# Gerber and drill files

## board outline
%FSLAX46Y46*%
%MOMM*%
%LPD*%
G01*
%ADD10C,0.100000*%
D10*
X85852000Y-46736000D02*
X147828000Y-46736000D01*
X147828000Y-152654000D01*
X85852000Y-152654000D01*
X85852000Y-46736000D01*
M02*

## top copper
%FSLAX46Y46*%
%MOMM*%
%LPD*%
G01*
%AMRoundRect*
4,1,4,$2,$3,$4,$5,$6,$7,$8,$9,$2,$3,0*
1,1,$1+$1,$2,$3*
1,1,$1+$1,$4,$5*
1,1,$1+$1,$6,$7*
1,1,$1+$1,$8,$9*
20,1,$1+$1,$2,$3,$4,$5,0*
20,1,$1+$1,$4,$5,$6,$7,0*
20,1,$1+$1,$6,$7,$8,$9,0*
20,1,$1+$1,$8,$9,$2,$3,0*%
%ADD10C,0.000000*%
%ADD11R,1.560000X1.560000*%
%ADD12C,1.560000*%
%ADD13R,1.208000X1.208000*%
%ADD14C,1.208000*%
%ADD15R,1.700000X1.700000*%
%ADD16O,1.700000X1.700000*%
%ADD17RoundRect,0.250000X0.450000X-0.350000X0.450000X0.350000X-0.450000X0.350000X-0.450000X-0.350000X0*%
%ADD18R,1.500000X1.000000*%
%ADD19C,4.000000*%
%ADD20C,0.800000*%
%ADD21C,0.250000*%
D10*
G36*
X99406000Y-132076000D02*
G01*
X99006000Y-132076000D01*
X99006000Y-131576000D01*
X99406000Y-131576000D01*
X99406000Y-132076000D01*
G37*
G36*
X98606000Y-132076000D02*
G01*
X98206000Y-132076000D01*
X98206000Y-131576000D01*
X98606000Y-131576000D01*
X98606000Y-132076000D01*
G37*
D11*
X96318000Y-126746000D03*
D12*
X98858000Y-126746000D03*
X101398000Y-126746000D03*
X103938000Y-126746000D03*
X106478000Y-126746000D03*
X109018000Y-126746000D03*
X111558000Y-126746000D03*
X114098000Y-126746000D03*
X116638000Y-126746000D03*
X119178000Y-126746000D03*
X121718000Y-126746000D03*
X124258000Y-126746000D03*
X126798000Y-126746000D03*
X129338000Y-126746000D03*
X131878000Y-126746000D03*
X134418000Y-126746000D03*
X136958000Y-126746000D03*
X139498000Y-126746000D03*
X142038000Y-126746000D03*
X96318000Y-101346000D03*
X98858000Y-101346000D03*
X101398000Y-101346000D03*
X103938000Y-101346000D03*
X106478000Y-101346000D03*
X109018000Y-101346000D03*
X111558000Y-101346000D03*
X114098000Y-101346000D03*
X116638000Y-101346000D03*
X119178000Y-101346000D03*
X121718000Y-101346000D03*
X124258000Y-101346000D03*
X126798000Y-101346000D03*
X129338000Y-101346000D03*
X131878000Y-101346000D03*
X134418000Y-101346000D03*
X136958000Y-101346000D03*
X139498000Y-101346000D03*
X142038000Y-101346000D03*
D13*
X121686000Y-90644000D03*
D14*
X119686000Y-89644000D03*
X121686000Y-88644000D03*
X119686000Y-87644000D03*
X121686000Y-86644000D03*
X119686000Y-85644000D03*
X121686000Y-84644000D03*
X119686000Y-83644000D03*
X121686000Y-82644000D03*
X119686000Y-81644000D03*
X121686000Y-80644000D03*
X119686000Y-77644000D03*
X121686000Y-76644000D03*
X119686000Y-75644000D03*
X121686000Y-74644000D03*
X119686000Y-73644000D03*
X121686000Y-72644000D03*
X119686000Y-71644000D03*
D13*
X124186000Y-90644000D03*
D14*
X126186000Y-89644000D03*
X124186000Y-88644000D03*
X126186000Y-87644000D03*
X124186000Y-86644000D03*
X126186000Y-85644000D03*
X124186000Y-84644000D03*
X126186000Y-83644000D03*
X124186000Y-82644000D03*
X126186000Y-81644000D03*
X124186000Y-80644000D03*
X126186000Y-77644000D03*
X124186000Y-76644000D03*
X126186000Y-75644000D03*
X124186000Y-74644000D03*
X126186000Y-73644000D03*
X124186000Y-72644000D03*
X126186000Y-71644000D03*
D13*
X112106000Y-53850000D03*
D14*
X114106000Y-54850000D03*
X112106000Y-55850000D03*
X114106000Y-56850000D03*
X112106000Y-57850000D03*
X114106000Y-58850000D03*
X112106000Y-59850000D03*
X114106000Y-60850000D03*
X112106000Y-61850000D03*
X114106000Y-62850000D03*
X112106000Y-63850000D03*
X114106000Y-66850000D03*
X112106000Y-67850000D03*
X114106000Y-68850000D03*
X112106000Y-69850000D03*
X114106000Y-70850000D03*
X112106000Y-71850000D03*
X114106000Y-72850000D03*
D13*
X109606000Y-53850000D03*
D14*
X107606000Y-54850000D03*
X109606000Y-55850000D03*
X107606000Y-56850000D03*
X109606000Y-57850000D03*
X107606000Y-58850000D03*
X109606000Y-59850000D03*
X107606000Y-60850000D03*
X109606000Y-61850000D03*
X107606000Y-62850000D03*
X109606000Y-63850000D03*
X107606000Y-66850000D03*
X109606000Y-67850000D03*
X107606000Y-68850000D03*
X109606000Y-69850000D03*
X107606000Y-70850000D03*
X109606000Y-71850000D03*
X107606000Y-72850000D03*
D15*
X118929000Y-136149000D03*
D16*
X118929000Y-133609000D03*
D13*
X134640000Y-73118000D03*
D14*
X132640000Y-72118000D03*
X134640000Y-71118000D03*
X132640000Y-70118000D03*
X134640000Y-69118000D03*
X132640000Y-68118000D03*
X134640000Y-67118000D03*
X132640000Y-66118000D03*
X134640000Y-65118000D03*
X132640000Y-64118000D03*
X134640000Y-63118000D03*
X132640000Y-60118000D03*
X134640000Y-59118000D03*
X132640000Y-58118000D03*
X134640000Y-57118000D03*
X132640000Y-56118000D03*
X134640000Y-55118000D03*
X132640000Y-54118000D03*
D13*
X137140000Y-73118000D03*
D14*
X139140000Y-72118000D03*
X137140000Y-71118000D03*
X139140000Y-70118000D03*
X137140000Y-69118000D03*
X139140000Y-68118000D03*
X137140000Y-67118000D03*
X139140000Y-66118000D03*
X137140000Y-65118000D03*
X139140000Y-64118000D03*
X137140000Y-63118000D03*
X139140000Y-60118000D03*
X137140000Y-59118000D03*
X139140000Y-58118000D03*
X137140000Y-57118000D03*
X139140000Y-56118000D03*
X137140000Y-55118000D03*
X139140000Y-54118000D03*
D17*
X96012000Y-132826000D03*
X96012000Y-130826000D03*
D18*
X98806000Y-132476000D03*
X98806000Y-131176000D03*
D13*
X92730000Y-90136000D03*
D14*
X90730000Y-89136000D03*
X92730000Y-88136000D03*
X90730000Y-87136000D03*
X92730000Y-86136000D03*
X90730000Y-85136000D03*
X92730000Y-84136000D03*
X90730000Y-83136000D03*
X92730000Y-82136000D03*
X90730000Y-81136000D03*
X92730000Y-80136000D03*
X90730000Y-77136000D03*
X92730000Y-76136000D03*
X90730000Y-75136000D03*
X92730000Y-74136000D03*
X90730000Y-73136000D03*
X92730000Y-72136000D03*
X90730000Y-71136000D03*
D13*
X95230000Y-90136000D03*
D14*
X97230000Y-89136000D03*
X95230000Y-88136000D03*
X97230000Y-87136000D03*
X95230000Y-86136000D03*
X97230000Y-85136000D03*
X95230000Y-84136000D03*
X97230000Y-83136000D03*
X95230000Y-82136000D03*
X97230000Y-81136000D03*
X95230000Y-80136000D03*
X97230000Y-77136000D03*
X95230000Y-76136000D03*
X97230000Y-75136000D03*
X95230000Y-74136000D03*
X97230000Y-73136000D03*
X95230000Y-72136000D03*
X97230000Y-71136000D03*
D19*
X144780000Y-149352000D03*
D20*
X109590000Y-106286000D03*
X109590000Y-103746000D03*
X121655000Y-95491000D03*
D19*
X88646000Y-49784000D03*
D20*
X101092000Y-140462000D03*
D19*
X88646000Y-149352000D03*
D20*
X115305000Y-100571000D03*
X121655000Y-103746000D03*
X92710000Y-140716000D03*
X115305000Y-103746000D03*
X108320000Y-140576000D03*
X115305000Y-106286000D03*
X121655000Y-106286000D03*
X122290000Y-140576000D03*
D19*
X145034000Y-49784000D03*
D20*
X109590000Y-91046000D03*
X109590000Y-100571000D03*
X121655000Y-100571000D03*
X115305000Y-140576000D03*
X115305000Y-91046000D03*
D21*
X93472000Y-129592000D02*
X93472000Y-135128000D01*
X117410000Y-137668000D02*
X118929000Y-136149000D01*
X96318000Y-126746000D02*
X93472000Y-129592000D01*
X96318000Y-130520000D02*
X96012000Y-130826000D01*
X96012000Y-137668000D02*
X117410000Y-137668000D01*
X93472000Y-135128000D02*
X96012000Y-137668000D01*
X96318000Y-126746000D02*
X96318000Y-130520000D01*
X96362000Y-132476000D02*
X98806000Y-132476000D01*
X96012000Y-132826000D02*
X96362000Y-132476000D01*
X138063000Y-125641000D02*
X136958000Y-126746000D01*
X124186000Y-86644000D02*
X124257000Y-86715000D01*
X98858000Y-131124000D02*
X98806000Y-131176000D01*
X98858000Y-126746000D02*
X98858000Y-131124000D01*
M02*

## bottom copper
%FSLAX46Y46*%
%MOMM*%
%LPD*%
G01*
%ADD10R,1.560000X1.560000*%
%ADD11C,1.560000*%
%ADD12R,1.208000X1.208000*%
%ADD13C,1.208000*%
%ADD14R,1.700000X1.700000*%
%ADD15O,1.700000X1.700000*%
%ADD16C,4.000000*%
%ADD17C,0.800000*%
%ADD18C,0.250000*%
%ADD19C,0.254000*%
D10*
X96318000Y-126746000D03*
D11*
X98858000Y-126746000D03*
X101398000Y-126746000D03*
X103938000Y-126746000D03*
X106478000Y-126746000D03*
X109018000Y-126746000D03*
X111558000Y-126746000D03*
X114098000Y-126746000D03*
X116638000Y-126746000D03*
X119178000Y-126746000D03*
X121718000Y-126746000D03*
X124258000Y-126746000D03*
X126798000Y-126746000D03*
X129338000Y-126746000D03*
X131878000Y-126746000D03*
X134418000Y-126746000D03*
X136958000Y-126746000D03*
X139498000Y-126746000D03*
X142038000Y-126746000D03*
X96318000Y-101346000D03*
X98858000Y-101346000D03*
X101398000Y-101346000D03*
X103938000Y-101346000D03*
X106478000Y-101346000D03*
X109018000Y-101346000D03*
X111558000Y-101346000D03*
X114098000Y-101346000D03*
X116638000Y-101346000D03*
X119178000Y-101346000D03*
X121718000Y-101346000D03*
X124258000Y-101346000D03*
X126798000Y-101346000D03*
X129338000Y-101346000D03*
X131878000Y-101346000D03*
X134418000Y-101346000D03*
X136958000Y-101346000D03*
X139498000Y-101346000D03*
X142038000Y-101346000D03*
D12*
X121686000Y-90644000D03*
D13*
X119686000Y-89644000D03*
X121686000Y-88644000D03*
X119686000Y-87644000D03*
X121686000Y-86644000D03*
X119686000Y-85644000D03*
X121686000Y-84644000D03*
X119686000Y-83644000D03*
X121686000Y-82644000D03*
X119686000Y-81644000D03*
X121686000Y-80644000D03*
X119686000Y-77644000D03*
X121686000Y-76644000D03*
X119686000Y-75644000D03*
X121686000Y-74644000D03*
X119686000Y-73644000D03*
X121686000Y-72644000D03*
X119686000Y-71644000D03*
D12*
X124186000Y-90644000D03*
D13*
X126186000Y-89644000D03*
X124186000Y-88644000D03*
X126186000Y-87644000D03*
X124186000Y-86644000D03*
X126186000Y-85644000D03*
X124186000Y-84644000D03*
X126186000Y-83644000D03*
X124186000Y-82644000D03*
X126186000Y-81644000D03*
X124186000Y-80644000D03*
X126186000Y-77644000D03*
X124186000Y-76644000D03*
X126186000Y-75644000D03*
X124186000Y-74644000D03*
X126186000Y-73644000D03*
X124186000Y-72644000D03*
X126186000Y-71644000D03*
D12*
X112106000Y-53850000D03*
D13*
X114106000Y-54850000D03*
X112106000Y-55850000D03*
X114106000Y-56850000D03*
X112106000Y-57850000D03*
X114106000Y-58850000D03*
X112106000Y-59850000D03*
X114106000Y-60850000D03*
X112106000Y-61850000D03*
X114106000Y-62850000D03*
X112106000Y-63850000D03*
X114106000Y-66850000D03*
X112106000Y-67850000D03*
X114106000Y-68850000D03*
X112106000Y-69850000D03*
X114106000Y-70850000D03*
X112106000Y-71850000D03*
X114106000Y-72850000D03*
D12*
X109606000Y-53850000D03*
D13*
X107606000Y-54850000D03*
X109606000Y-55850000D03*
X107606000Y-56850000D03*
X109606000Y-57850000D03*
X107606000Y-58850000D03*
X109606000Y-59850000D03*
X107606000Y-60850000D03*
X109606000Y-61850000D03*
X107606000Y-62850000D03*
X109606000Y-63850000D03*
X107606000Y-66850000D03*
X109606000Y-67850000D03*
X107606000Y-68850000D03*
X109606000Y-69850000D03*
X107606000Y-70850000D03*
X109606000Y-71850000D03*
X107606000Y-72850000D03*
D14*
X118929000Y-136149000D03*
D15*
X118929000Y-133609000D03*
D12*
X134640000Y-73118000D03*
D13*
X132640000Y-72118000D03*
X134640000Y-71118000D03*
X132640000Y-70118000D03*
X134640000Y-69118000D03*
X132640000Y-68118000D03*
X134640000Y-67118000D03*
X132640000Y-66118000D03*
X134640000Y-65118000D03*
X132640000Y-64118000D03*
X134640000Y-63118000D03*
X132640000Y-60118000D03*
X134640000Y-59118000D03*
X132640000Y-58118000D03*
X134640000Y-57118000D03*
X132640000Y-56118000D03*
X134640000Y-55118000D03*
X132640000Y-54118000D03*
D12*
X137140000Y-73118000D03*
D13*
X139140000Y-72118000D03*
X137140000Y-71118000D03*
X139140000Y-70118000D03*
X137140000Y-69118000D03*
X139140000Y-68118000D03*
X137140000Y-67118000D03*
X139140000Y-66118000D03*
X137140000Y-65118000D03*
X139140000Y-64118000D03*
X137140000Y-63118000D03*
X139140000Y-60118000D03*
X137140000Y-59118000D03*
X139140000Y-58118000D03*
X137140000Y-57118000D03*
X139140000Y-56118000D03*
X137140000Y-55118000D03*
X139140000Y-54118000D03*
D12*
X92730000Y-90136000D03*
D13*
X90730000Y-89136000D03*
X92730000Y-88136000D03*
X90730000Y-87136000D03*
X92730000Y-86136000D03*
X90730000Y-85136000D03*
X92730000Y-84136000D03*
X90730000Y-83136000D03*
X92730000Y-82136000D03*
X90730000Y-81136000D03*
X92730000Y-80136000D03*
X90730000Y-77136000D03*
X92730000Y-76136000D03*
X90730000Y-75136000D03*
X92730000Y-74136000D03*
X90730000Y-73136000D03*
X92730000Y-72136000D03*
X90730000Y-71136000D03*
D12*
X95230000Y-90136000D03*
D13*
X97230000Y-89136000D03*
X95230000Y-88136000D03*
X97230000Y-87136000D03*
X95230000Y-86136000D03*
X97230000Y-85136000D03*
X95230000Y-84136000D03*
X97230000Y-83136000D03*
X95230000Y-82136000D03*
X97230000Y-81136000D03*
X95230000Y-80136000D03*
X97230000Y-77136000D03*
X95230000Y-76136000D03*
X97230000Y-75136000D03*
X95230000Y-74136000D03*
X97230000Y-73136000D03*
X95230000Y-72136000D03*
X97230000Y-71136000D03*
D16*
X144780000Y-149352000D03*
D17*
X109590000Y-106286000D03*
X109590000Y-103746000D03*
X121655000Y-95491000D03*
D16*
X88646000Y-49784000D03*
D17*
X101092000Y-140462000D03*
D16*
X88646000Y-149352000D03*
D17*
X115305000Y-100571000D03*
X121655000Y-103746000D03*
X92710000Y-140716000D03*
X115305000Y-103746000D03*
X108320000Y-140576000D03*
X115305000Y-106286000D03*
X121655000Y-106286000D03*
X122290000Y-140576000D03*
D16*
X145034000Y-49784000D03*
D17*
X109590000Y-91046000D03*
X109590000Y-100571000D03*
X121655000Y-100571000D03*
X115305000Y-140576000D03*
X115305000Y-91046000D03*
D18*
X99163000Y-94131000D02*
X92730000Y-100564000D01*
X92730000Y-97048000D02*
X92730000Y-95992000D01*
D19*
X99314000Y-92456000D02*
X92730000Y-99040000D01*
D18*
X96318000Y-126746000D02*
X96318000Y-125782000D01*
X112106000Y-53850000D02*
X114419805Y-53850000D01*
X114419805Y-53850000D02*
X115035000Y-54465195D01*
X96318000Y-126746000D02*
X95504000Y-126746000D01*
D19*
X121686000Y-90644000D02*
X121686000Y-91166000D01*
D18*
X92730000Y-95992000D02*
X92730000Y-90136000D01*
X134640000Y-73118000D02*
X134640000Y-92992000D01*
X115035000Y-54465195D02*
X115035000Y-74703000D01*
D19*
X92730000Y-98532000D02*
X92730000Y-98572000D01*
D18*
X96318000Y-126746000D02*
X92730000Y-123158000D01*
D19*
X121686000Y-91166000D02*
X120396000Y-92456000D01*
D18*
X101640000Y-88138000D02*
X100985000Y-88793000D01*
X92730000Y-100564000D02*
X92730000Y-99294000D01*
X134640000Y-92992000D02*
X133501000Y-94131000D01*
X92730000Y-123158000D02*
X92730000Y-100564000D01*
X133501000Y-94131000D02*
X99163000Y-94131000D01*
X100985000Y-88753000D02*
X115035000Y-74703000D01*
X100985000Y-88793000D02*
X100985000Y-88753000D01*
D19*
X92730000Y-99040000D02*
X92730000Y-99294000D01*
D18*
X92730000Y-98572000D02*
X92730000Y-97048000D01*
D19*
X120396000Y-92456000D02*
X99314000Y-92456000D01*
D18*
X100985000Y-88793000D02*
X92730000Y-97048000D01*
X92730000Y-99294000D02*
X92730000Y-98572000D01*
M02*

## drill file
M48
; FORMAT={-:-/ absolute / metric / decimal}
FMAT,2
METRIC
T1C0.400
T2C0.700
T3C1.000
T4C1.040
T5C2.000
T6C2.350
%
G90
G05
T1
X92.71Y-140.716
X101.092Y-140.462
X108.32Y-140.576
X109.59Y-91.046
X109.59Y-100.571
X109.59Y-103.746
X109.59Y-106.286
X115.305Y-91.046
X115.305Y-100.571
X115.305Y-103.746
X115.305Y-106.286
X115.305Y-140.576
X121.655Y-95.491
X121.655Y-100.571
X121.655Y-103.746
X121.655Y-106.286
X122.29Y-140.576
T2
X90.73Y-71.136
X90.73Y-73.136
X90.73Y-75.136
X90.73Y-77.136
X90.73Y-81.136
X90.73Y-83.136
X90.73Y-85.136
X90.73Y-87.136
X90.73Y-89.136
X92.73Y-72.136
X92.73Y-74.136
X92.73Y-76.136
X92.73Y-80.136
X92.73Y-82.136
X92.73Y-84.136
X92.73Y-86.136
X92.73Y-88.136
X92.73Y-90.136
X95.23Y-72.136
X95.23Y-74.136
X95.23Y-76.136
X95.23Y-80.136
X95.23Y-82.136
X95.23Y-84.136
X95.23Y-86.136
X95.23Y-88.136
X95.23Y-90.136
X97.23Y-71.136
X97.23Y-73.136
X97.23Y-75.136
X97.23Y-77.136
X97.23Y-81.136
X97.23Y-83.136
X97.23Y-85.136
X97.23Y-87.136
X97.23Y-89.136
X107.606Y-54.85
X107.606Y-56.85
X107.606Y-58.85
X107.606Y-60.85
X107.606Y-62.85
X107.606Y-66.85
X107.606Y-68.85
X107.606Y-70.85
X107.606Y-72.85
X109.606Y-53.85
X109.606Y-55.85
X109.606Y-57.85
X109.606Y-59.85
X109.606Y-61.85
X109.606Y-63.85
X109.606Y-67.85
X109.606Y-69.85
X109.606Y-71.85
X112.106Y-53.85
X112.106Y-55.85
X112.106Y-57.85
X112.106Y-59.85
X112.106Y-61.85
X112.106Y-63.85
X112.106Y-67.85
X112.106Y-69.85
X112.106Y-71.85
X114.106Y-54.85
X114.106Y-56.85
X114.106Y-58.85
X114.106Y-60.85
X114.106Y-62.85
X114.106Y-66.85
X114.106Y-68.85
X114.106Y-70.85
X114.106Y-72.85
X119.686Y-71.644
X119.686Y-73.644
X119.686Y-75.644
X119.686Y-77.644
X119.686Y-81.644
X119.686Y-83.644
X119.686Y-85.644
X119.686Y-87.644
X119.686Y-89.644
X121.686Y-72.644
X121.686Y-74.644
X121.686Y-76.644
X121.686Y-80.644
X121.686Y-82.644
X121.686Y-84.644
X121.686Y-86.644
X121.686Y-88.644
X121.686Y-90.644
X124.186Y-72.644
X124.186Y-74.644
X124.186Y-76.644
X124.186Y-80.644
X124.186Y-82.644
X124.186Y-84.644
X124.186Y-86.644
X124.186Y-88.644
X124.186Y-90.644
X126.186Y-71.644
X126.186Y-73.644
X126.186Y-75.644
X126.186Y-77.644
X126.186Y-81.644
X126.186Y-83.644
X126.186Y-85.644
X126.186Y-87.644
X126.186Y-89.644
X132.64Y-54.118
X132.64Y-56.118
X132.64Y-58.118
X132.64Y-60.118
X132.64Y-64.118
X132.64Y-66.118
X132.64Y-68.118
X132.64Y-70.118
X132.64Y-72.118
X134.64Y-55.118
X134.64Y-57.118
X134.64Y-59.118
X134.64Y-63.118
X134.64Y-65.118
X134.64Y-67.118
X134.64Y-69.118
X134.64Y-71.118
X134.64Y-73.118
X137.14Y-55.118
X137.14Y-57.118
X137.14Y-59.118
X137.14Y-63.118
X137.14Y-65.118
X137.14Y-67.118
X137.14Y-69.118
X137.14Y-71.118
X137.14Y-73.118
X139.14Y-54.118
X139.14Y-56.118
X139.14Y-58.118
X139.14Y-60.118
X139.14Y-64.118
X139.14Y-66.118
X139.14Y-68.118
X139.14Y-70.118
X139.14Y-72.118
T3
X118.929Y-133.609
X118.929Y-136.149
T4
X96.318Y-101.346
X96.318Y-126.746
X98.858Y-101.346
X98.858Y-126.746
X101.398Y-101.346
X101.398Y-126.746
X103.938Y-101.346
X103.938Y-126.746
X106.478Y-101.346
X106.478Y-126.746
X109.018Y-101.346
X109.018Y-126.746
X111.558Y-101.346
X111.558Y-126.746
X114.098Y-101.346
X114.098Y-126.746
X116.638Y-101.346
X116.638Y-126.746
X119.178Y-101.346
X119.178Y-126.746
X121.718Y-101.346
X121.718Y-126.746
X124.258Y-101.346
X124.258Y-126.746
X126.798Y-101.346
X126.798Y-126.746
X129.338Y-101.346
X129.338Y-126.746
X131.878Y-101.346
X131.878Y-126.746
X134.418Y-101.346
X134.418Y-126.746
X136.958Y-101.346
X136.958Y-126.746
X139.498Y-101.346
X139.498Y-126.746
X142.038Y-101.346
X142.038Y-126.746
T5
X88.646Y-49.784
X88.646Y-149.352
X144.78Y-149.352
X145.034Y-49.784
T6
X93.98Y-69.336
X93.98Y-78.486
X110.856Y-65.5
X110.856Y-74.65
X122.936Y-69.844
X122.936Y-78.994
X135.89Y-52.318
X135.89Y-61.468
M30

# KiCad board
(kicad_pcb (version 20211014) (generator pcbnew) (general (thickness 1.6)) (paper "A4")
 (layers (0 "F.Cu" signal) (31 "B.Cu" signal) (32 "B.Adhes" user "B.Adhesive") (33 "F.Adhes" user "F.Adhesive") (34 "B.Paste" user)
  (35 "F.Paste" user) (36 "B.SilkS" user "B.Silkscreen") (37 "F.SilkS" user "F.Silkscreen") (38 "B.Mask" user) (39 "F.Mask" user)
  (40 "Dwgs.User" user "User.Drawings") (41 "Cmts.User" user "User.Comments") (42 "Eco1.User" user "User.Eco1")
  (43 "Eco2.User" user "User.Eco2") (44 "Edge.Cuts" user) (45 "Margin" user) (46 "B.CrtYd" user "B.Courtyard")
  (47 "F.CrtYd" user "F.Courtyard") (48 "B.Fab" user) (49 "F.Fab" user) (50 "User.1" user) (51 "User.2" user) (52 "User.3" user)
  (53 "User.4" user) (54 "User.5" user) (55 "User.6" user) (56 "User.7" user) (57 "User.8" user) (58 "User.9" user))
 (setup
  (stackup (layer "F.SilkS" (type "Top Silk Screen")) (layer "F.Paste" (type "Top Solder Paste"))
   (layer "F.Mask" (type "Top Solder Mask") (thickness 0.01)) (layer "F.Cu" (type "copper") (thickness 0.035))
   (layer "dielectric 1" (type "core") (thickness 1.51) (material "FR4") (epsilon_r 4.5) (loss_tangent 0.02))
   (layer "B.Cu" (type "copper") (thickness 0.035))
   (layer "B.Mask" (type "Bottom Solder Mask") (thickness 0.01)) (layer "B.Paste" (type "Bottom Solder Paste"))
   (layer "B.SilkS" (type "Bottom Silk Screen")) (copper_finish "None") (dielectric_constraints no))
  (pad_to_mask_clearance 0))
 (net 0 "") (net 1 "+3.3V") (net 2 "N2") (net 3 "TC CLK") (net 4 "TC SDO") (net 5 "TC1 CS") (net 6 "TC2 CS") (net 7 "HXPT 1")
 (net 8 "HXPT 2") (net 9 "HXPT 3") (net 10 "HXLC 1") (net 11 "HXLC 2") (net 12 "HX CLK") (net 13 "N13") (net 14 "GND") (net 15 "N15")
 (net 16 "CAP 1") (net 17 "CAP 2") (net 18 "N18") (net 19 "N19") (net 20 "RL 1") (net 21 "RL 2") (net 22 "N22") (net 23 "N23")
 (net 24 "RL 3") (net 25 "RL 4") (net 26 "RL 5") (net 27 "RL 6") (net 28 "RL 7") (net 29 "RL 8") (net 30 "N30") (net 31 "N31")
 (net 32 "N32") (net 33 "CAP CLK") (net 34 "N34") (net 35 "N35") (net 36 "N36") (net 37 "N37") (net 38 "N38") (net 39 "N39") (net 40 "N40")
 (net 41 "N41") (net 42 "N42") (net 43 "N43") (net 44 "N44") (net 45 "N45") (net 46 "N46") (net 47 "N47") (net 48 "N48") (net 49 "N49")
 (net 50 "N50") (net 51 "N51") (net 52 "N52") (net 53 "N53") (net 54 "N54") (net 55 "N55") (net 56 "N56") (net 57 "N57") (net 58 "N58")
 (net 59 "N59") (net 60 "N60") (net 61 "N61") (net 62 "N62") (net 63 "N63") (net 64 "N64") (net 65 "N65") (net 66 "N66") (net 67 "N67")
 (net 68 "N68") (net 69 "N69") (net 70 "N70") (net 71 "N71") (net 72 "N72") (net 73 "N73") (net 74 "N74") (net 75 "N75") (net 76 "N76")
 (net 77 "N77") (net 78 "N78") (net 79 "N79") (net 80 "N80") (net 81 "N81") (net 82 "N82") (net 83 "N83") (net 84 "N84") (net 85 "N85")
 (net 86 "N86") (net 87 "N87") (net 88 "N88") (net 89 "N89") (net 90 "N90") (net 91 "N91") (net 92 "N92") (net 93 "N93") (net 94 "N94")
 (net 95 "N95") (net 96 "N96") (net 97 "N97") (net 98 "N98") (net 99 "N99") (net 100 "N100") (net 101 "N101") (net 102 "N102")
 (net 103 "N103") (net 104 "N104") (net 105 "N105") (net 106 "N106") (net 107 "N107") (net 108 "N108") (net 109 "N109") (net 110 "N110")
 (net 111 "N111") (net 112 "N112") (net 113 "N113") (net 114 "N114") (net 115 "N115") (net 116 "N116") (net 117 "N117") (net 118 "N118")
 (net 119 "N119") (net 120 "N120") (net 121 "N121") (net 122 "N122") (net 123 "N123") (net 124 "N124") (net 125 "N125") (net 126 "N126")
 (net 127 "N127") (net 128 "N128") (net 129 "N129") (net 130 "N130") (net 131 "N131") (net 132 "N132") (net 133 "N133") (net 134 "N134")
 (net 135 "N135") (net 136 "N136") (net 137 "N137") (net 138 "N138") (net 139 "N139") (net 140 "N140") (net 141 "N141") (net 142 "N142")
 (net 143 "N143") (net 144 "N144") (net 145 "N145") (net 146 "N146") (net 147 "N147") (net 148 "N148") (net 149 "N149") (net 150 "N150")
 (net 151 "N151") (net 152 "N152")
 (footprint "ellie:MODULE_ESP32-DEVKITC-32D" (layer "F.Cu") (at 116.078 114.046 90)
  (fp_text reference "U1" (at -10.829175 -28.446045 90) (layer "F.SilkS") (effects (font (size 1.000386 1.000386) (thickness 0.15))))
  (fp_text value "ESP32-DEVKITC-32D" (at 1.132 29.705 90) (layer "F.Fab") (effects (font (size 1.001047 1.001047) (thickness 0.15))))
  (pad "1" thru_hole rect locked (at -12.7 -19.76 90) (size 1.56 1.56) (drill 1.04) (layers *.Cu *.Mask) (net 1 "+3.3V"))
  (pad "2" thru_hole circle locked (at -12.7 -17.22 90) (size 1.56 1.56) (drill 1.04) (layers *.Cu *.Mask) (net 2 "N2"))
  (pad "3" thru_hole circle locked (at -12.7 -14.68 90) (size 1.56 1.56) (drill 1.04) (layers *.Cu *.Mask) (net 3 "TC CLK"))
  (pad "4" thru_hole circle locked (at -12.7 -12.14 90) (size 1.56 1.56) (drill 1.04) (layers *.Cu *.Mask) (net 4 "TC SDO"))
  (pad "5" thru_hole circle locked (at -12.7 -9.6 90) (size 1.56 1.56) (drill 1.04) (layers *.Cu *.Mask) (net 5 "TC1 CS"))
  (pad "6" thru_hole circle locked (at -12.7 -7.06 90) (size 1.56 1.56) (drill 1.04) (layers *.Cu *.Mask) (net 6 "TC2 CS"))
  (pad "7" thru_hole circle locked (at -12.7 -4.52 90) (size 1.56 1.56) (drill 1.04) (layers *.Cu *.Mask) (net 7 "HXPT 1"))
  (pad "8" thru_hole circle locked (at -12.7 -1.98 90) (size 1.56 1.56) (drill 1.04) (layers *.Cu *.Mask) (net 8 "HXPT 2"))
  (pad "9" thru_hole circle locked (at -12.7 0.56 90) (size 1.56 1.56) (drill 1.04) (layers *.Cu *.Mask) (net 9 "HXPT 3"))
  (pad "10" thru_hole circle locked (at -12.7 3.1 90) (size 1.56 1.56) (drill 1.04) (layers *.Cu *.Mask) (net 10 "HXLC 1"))
  (pad "11" thru_hole circle locked (at -12.7 5.64 90) (size 1.56 1.56) (drill 1.04) (layers *.Cu *.Mask) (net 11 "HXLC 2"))
  (pad "12" thru_hole circle locked (at -12.7 8.18 90) (size 1.56 1.56) (drill 1.04) (layers *.Cu *.Mask) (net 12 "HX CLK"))
  (pad "13" thru_hole circle locked (at -12.7 10.72 90) (size 1.56 1.56) (drill 1.04) (layers *.Cu *.Mask) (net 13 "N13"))
  (pad "14" thru_hole circle locked (at -12.7 13.26 90) (size 1.56 1.56) (drill 1.04) (layers *.Cu *.Mask) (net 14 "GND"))
  (pad "15" thru_hole circle locked (at -12.7 15.8 90) (size 1.56 1.56) (drill 1.04) (layers *.Cu *.Mask) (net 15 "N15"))
  (pad "16" thru_hole circle locked (at -12.7 18.34 90) (size 1.56 1.56) (drill 1.04) (layers *.Cu *.Mask) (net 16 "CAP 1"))
  (pad "17" thru_hole circle locked (at -12.7 20.88 90) (size 1.56 1.56) (drill 1.04) (layers *.Cu *.Mask) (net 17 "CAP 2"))
  (pad "18" thru_hole circle locked (at -12.7 23.42 90) (size 1.56 1.56) (drill 1.04) (layers *.Cu *.Mask) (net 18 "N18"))
  (pad "19" thru_hole circle locked (at -12.7 25.96 90) (size 1.56 1.56) (drill 1.04) (layers *.Cu *.Mask) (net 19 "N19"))
  (pad "20" thru_hole circle locked (at 12.7 -19.76 90) (size 1.56 1.56) (drill 1.04) (layers *.Cu *.Mask) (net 14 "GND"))
  (pad "21" thru_hole circle locked (at 12.7 -17.22 90) (size 1.56 1.56) (drill 1.04) (layers *.Cu *.Mask) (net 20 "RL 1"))
  (pad "22" thru_hole circle locked (at 12.7 -14.68 90) (size 1.56 1.56) (drill 1.04) (layers *.Cu *.Mask) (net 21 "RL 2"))
  (pad "23" thru_hole circle locked (at 12.7 -12.14 90) (size 1.56 1.56) (drill 1.04) (layers *.Cu *.Mask) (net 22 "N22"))
  (pad "24" thru_hole circle locked (at 12.7 -9.6 90) (size 1.56 1.56) (drill 1.04) (layers *.Cu *.Mask) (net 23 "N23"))
  (pad "25" thru_hole circle locked (at 12.7 -7.06 90) (size 1.56 1.56) (drill 1.04) (layers *.Cu *.Mask) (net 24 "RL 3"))
  (pad "26" thru_hole circle locked (at 12.7 -4.52 90) (size 1.56 1.56) (drill 1.04) (layers *.Cu *.Mask) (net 14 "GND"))
  (pad "27" thru_hole circle locked (at 12.7 -1.98 90) (size 1.56 1.56) (drill 1.04) (layers *.Cu *.Mask) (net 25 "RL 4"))
  (pad "28" thru_hole circle locked (at 12.7 0.56 90) (size 1.56 1.56) (drill 1.04) (layers *.Cu *.Mask) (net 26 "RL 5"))
  (pad "29" thru_hole circle locked (at 12.7 3.1 90) (size 1.56 1.56) (drill 1.04) (layers *.Cu *.Mask) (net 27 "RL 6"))
  (pad "30" thru_hole circle locked (at 12.7 5.64 90) (size 1.56 1.56) (drill 1.04) (layers *.Cu *.Mask) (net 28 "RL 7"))
  (pad "31" thru_hole circle locked (at 12.7 8.18 90) (size 1.56 1.56) (drill 1.04) (layers *.Cu *.Mask) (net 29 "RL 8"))
  (pad "32" thru_hole circle locked (at 12.7 10.72 90) (size 1.56 1.56) (drill 1.04) (layers *.Cu *.Mask) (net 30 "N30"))
  (pad "33" thru_hole circle locked (at 12.7 13.26 90) (size 1.56 1.56) (drill 1.04) (layers *.Cu *.Mask) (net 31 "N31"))
  (pad "34" thru_hole circle locked (at 12.7 15.8 90) (size 1.56 1.56) (drill 1.04) (layers *.Cu *.Mask) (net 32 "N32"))
  (pad "35" thru_hole circle locked (at 12.7 18.34 90) (size 1.56 1.56) (drill 1.04) (layers *.Cu *.Mask) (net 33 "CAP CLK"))
  (pad "36" thru_hole circle locked (at 12.7 20.88 90) (size 1.56 1.56) (drill 1.04) (layers *.Cu *.Mask) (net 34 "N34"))
  (pad "37" thru_hole circle locked (at 12.7 23.42 90) (size 1.56 1.56) (drill 1.04) (layers *.Cu *.Mask) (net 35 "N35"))
  (pad "38" thru_hole circle locked (at 12.7 25.96 90) (size 1.56 1.56) (drill 1.04) (layers *.Cu *.Mask) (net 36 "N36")))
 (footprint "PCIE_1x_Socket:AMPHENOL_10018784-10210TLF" (layer "F.Cu") (at 122.936 78.994 90)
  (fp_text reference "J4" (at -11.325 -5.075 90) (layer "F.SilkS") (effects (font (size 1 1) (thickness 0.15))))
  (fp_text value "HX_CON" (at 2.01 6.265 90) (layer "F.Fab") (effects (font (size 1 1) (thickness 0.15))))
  (pad "" np_thru_hole circle locked (at 9.15 0 90) (size 2.35 2.35) (drill 2.35) (layers *.Cu *.Mask))
  (pad "" np_thru_hole circle locked (at 0 0 90) (size 2.35 2.35) (drill 2.35) (layers *.Cu *.Mask))
  (pad "A1" thru_hole rect locked (at -11.65 -1.25 90) (size 1.208 1.208) (drill 0.7) (layers *.Cu *.Mask) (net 1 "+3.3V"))
  (pad "A2" thru_hole circle locked (at -10.65 -3.25 90) (size 1.208 1.208) (drill 0.7) (layers *.Cu *.Mask) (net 14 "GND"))
  (pad "A3" thru_hole circle locked (at -9.65 -1.25 90) (size 1.208 1.208) (drill 0.7) (layers *.Cu *.Mask) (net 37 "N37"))
  (pad "A4" thru_hole circle locked (at -8.65 -3.25 90) (size 1.208 1.208) (drill 0.7) (layers *.Cu *.Mask) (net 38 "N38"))
  (pad "A5" thru_hole circle locked (at -7.65 -1.25 90) (size 1.208 1.208) (drill 0.7) (layers *.Cu *.Mask) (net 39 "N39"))
  (pad "A6" thru_hole circle locked (at -6.65 -3.25 90) (size 1.208 1.208) (drill 0.7) (layers *.Cu *.Mask) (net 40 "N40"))
  (pad "A7" thru_hole circle locked (at -5.65 -1.25 90) (size 1.208 1.208) (drill 0.7) (layers *.Cu *.Mask) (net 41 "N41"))
  (pad "A8" thru_hole circle locked (at -4.65 -3.25 90) (size 1.208 1.208) (drill 0.7) (layers *.Cu *.Mask) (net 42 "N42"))
  (pad "A9" thru_hole circle locked (at -3.65 -1.25 90) (size 1.208 1.208) (drill 0.7) (layers *.Cu *.Mask) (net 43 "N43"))
  (pad "A10" thru_hole circle locked (at -2.65 -3.25 90) (size 1.208 1.208) (drill 0.7) (layers *.Cu *.Mask) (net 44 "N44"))
  (pad "A11" thru_hole circle locked (at -1.65 -1.25 90) (size 1.208 1.208) (drill 0.7) (layers *.Cu *.Mask) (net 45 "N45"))
  (pad "A12" thru_hole circle locked (at 1.35 -3.25 90) (size 1.208 1.208) (drill 0.7) (layers *.Cu *.Mask) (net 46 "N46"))
  (pad "A13" thru_hole circle locked (at 2.35 -1.25 90) (size 1.208 1.208) (drill 0.7) (layers *.Cu *.Mask) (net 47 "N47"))
  (pad "A14" thru_hole circle locked (at 3.35 -3.25 90) (size 1.208 1.208) (drill 0.7) (layers *.Cu *.Mask) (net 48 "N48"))
  (pad "A15" thru_hole circle locked (at 4.35 -1.25 90) (size 1.208 1.208) (drill 0.7) (layers *.Cu *.Mask) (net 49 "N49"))
  (pad "A16" thru_hole circle locked (at 5.35 -3.25 90) (size 1.208 1.208) (drill 0.7) (layers *.Cu *.Mask) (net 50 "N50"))
  (pad "A17" thru_hole circle locked (at 6.35 -1.25 90) (size 1.208 1.208) (drill 0.7) (layers *.Cu *.Mask) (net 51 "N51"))
  (pad "A18" thru_hole circle locked (at 7.35 -3.25 90) (size 1.208 1.208) (drill 0.7) (layers *.Cu *.Mask) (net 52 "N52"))
  (pad "B1" thru_hole rect locked (at -11.65 1.25 90) (size 1.208 1.208) (drill 0.7) (layers *.Cu *.Mask) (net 7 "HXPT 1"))
  (pad "B2" thru_hole circle locked (at -10.65 3.25 90) (size 1.208 1.208) (drill 0.7) (layers *.Cu *.Mask) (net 8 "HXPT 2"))
  (pad "B3" thru_hole circle locked (at -9.65 1.25 90) (size 1.208 1.208) (drill 0.7) (layers *.Cu *.Mask) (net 9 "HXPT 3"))
  (pad "B4" thru_hole circle locked (at -8.65 3.25 90) (size 1.208 1.208) (drill 0.7) (layers *.Cu *.Mask) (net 10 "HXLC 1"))
  (pad "B5" thru_hole circle locked (at -7.65 1.25 90) (size 1.208 1.208) (drill 0.7) (layers *.Cu *.Mask) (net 11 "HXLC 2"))
  (pad "B6" thru_hole circle locked (at -6.65 3.25 90) (size 1.208 1.208) (drill 0.7) (layers *.Cu *.Mask) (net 12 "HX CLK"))
  (pad "B7" thru_hole circle locked (at -5.65 1.25 90) (size 1.208 1.208) (drill 0.7) (layers *.Cu *.Mask) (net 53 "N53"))
  (pad "B8" thru_hole circle locked (at -4.65 3.25 90) (size 1.208 1.208) (drill 0.7) (layers *.Cu *.Mask) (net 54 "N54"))
  (pad "B9" thru_hole circle locked (at -3.65 1.25 90) (size 1.208 1.208) (drill 0.7) (layers *.Cu *.Mask) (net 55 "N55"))
  (pad "B10" thru_hole circle locked (at -2.65 3.25 90) (size 1.208 1.208) (drill 0.7) (layers *.Cu *.Mask) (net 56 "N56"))
  (pad "B11" thru_hole circle locked (at -1.65 1.25 90) (size 1.208 1.208) (drill 0.7) (layers *.Cu *.Mask) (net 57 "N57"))
  (pad "B12" thru_hole circle locked (at 1.35 3.25 90) (size 1.208 1.208) (drill 0.7) (layers *.Cu *.Mask) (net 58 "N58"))
  (pad "B13" thru_hole circle locked (at 2.35 1.25 90) (size 1.208 1.208) (drill 0.7) (layers *.Cu *.Mask) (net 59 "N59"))
  (pad "B14" thru_hole circle locked (at 3.35 3.25 90) (size 1.208 1.208) (drill 0.7) (layers *.Cu *.Mask) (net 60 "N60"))
  (pad "B15" thru_hole circle locked (at 4.35 1.25 90) (size 1.208 1.208) (drill 0.7) (layers *.Cu *.Mask) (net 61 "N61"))
  (pad "B16" thru_hole circle locked (at 5.35 3.25 90) (size 1.208 1.208) (drill 0.7) (layers *.Cu *.Mask) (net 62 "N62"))
  (pad "B17" thru_hole circle locked (at 6.35 1.25 90) (size 1.208 1.208) (drill 0.7) (layers *.Cu *.Mask) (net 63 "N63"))
  (pad "B18" thru_hole circle locked (at 7.35 3.25 90) (size 1.208 1.208) (drill 0.7) (layers *.Cu *.Mask) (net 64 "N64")))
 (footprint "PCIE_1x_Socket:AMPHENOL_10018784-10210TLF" (layer "F.Cu") (at 110.856 65.5 -90)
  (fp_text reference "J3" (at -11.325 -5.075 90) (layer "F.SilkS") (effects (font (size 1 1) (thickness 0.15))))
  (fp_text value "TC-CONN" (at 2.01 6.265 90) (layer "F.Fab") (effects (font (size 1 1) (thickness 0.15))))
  (pad "" np_thru_hole circle locked (at 0 0 270) (size 2.35 2.35) (drill 2.35) (layers *.Cu *.Mask))
  (pad "" np_thru_hole circle locked (at 9.15 0 270) (size 2.35 2.35) (drill 2.35) (layers *.Cu *.Mask))
  (pad "A1" thru_hole rect locked (at -11.65 -1.25 270) (size 1.208 1.208) (drill 0.7) (layers *.Cu *.Mask) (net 1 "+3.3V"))
  (pad "A2" thru_hole circle locked (at -10.65 -3.25 270) (size 1.208 1.208) (drill 0.7) (layers *.Cu *.Mask) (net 14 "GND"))
  (pad "A3" thru_hole circle locked (at -9.65 -1.25 270) (size 1.208 1.208) (drill 0.7) (layers *.Cu *.Mask) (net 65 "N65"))
  (pad "A4" thru_hole circle locked (at -8.65 -3.25 270) (size 1.208 1.208) (drill 0.7) (layers *.Cu *.Mask) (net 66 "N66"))
  (pad "A5" thru_hole circle locked (at -7.65 -1.25 270) (size 1.208 1.208) (drill 0.7) (layers *.Cu *.Mask) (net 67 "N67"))
  (pad "A6" thru_hole circle locked (at -6.65 -3.25 270) (size 1.208 1.208) (drill 0.7) (layers *.Cu *.Mask) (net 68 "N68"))
  (pad "A7" thru_hole circle locked (at -5.65 -1.25 270) (size 1.208 1.208) (drill 0.7) (layers *.Cu *.Mask) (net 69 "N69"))
  (pad "A8" thru_hole circle locked (at -4.65 -3.25 270) (size 1.208 1.208) (drill 0.7) (layers *.Cu *.Mask) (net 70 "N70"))
  (pad "A9" thru_hole circle locked (at -3.65 -1.25 270) (size 1.208 1.208) (drill 0.7) (layers *.Cu *.Mask) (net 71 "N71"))
  (pad "A10" thru_hole circle locked (at -2.65 -3.25 270) (size 1.208 1.208) (drill 0.7) (layers *.Cu *.Mask) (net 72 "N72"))
  (pad "A11" thru_hole circle locked (at -1.65 -1.25 270) (size 1.208 1.208) (drill 0.7) (layers *.Cu *.Mask) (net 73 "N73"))
  (pad "A12" thru_hole circle locked (at 1.35 -3.25 270) (size 1.208 1.208) (drill 0.7) (layers *.Cu *.Mask) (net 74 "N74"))
  (pad "A13" thru_hole circle locked (at 2.35 -1.25 270) (size 1.208 1.208) (drill 0.7) (layers *.Cu *.Mask) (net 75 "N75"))
  (pad "A14" thru_hole circle locked (at 3.35 -3.25 270) (size 1.208 1.208) (drill 0.7) (layers *.Cu *.Mask) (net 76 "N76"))
  (pad "A15" thru_hole circle locked (at 4.35 -1.25 270) (size 1.208 1.208) (drill 0.7) (layers *.Cu *.Mask) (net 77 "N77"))
  (pad "A16" thru_hole circle locked (at 5.35 -3.25 270) (size 1.208 1.208) (drill 0.7) (layers *.Cu *.Mask) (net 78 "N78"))
  (pad "A17" thru_hole circle locked (at 6.35 -1.25 270) (size 1.208 1.208) (drill 0.7) (layers *.Cu *.Mask) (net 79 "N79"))
  (pad "A18" thru_hole circle locked (at 7.35 -3.25 270) (size 1.208 1.208) (drill 0.7) (layers *.Cu *.Mask) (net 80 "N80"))
  (pad "B1" thru_hole rect locked (at -11.65 1.25 270) (size 1.208 1.208) (drill 0.7) (layers *.Cu *.Mask) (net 6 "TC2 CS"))
  (pad "B2" thru_hole circle locked (at -10.65 3.25 270) (size 1.208 1.208) (drill 0.7) (layers *.Cu *.Mask) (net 5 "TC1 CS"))
  (pad "B3" thru_hole circle locked (at -9.65 1.25 270) (size 1.208 1.208) (drill 0.7) (layers *.Cu *.Mask) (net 4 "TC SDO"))
  (pad "B4" thru_hole circle locked (at -8.65 3.25 270) (size 1.208 1.208) (drill 0.7) (layers *.Cu *.Mask) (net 3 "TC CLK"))
  (pad "B5" thru_hole circle locked (at -7.65 1.25 270) (size 1.208 1.208) (drill 0.7) (layers *.Cu *.Mask) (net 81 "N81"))
  (pad "B6" thru_hole circle locked (at -6.65 3.25 270) (size 1.208 1.208) (drill 0.7) (layers *.Cu *.Mask) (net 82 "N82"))
  (pad "B7" thru_hole circle locked (at -5.65 1.25 270) (size 1.208 1.208) (drill 0.7) (layers *.Cu *.Mask) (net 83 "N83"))
  (pad "B8" thru_hole circle locked (at -4.65 3.25 270) (size 1.208 1.208) (drill 0.7) (layers *.Cu *.Mask) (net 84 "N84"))
  (pad "B9" thru_hole circle locked (at -3.65 1.25 270) (size 1.208 1.208) (drill 0.7) (layers *.Cu *.Mask) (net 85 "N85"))
  (pad "B10" thru_hole circle locked (at -2.65 3.25 270) (size 1.208 1.208) (drill 0.7) (layers *.Cu *.Mask) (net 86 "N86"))
  (pad "B11" thru_hole circle locked (at -1.65 1.25 270) (size 1.208 1.208) (drill 0.7) (layers *.Cu *.Mask) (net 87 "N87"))
  (pad "B12" thru_hole circle locked (at 1.35 3.25 270) (size 1.208 1.208) (drill 0.7) (layers *.Cu *.Mask) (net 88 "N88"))
  (pad "B13" thru_hole circle locked (at 2.35 1.25 270) (size 1.208 1.208) (drill 0.7) (layers *.Cu *.Mask) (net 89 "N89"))
  (pad "B14" thru_hole circle locked (at 3.35 3.25 270) (size 1.208 1.208) (drill 0.7) (layers *.Cu *.Mask) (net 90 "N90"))
  (pad "B15" thru_hole circle locked (at 4.35 1.25 270) (size 1.208 1.208) (drill 0.7) (layers *.Cu *.Mask) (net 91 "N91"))
  (pad "B16" thru_hole circle locked (at 5.35 3.25 270) (size 1.208 1.208) (drill 0.7) (layers *.Cu *.Mask) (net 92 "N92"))
  (pad "B17" thru_hole circle locked (at 6.35 1.25 270) (size 1.208 1.208) (drill 0.7) (layers *.Cu *.Mask) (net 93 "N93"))
  (pad "B18" thru_hole circle locked (at 7.35 3.25 270) (size 1.208 1.208) (drill 0.7) (layers *.Cu *.Mask) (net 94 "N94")))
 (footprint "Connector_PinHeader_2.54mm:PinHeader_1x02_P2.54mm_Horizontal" (layer "F.Cu") (at 118.929 136.149 180)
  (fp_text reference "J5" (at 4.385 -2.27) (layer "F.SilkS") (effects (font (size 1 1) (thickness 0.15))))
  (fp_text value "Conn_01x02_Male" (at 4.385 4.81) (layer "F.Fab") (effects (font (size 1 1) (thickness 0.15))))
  (pad "1" thru_hole rect (at 0 0 180) (size 1.7 1.7) (drill 1) (layers *.Cu *.Mask) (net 1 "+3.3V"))
  (pad "2" thru_hole oval (at 0 2.54 180) (size 1.7 1.7) (drill 1) (layers *.Cu *.Mask) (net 14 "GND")))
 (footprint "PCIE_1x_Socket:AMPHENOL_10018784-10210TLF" (layer "F.Cu") (at 135.89 61.468 90)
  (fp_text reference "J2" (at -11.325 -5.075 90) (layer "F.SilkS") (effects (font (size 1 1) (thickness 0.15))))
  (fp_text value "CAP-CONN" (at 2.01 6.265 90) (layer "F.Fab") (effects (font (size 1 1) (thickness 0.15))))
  (pad "" np_thru_hole circle locked (at 9.15 0 90) (size 2.35 2.35) (drill 2.35) (layers *.Cu *.Mask))
  (pad "" np_thru_hole circle locked (at 0 0 90) (size 2.35 2.35) (drill 2.35) (layers *.Cu *.Mask))
  (pad "A1" thru_hole rect locked (at -11.65 -1.25 90) (size 1.208 1.208) (drill 0.7) (layers *.Cu *.Mask) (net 1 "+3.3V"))
  (pad "A2" thru_hole circle locked (at -10.65 -3.25 90) (size 1.208 1.208) (drill 0.7) (layers *.Cu *.Mask) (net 14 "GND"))
  (pad "A3" thru_hole circle locked (at -9.65 -1.25 90) (size 1.208 1.208) (drill 0.7) (layers *.Cu *.Mask) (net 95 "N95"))
  (pad "A4" thru_hole circle locked (at -8.65 -3.25 90) (size 1.208 1.208) (drill 0.7) (layers *.Cu *.Mask) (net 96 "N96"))
  (pad "A5" thru_hole circle locked (at -7.65 -1.25 90) (size 1.208 1.208) (drill 0.7) (layers *.Cu *.Mask) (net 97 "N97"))
  (pad "A6" thru_hole circle locked (at -6.65 -3.25 90) (size 1.208 1.208) (drill 0.7) (layers *.Cu *.Mask) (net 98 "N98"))
  (pad "A7" thru_hole circle locked (at -5.65 -1.25 90) (size 1.208 1.208) (drill 0.7) (layers *.Cu *.Mask) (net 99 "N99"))
  (pad "A8" thru_hole circle locked (at -4.65 -3.25 90) (size 1.208 1.208) (drill 0.7) (layers *.Cu *.Mask) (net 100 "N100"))
  (pad "A9" thru_hole circle locked (at -3.65 -1.25 90) (size 1.208 1.208) (drill 0.7) (layers *.Cu *.Mask) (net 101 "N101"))
  (pad "A10" thru_hole circle locked (at -2.65 -3.25 90) (size 1.208 1.208) (drill 0.7) (layers *.Cu *.Mask) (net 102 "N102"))
  (pad "A11" thru_hole circle locked (at -1.65 -1.25 90) (size 1.208 1.208) (drill 0.7) (layers *.Cu *.Mask) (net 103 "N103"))
  (pad "A12" thru_hole circle locked (at 1.35 -3.25 90) (size 1.208 1.208) (drill 0.7) (layers *.Cu *.Mask) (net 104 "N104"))
  (pad "A13" thru_hole circle locked (at 2.35 -1.25 90) (size 1.208 1.208) (drill 0.7) (layers *.Cu *.Mask) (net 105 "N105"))
  (pad "A14" thru_hole circle locked (at 3.35 -3.25 90) (size 1.208 1.208) (drill 0.7) (layers *.Cu *.Mask) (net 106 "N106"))
  (pad "A15" thru_hole circle locked (at 4.35 -1.25 90) (size 1.208 1.208) (drill 0.7) (layers *.Cu *.Mask) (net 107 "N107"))
  (pad "A16" thru_hole circle locked (at 5.35 -3.25 90) (size 1.208 1.208) (drill 0.7) (layers *.Cu *.Mask) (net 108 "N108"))
  (pad "A17" thru_hole circle locked (at 6.35 -1.25 90) (size 1.208 1.208) (drill 0.7) (layers *.Cu *.Mask) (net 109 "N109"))
  (pad "A18" thru_hole circle locked (at 7.35 -3.25 90) (size 1.208 1.208) (drill 0.7) (layers *.Cu *.Mask) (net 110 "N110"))
  (pad "B1" thru_hole rect locked (at -11.65 1.25 90) (size 1.208 1.208) (drill 0.7) (layers *.Cu *.Mask) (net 16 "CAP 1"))
  (pad "B2" thru_hole circle locked (at -10.65 3.25 90) (size 1.208 1.208) (drill 0.7) (layers *.Cu *.Mask) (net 17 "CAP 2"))
  (pad "B3" thru_hole circle locked (at -9.65 1.25 90) (size 1.208 1.208) (drill 0.7) (layers *.Cu *.Mask) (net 33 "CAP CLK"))
  (pad "B4" thru_hole circle locked (at -8.65 3.25 90) (size 1.208 1.208) (drill 0.7) (layers *.Cu *.Mask) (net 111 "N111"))
  (pad "B5" thru_hole circle locked (at -7.65 1.25 90) (size 1.208 1.208) (drill 0.7) (layers *.Cu *.Mask) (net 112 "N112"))
  (pad "B6" thru_hole circle locked (at -6.65 3.25 90) (size 1.208 1.208) (drill 0.7) (layers *.Cu *.Mask) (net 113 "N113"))
  (pad "B7" thru_hole circle locked (at -5.65 1.25 90) (size 1.208 1.208) (drill 0.7) (layers *.Cu *.Mask) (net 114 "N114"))
  (pad "B8" thru_hole circle locked (at -4.65 3.25 90) (size 1.208 1.208) (drill 0.7) (layers *.Cu *.Mask) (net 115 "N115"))
  (pad "B9" thru_hole circle locked (at -3.65 1.25 90) (size 1.208 1.208) (drill 0.7) (layers *.Cu *.Mask) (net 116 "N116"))
  (pad "B10" thru_hole circle locked (at -2.65 3.25 90) (size 1.208 1.208) (drill 0.7) (layers *.Cu *.Mask) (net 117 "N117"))
  (pad "B11" thru_hole circle locked (at -1.65 1.25 90) (size 1.208 1.208) (drill 0.7) (layers *.Cu *.Mask) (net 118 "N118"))
  (pad "B12" thru_hole circle locked (at 1.35 3.25 90) (size 1.208 1.208) (drill 0.7) (layers *.Cu *.Mask) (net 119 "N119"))
  (pad "B13" thru_hole circle locked (at 2.35 1.25 90) (size 1.208 1.208) (drill 0.7) (layers *.Cu *.Mask) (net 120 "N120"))
  (pad "B14" thru_hole circle locked (at 3.35 3.25 90) (size 1.208 1.208) (drill 0.7) (layers *.Cu *.Mask) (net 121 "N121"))
  (pad "B15" thru_hole circle locked (at 4.35 1.25 90) (size 1.208 1.208) (drill 0.7) (layers *.Cu *.Mask) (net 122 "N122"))
  (pad "B16" thru_hole circle locked (at 5.35 3.25 90) (size 1.208 1.208) (drill 0.7) (layers *.Cu *.Mask) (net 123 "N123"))
  (pad "B17" thru_hole circle locked (at 6.35 1.25 90) (size 1.208 1.208) (drill 0.7) (layers *.Cu *.Mask) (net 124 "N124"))
  (pad "B18" thru_hole circle locked (at 7.35 3.25 90) (size 1.208 1.208) (drill 0.7) (layers *.Cu *.Mask) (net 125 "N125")))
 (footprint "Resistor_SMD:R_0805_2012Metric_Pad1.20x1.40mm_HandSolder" (layer "F.Cu") (at 96.012 131.826 90)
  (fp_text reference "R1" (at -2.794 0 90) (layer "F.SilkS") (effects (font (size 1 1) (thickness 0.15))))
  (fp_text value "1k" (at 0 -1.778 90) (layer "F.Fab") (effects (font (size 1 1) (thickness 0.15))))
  (pad "1" smd roundrect (at -1 0 90) (size 1.2 1.4) (layers "F.Cu" "F.Paste" "F.Mask") (roundrect_rratio 0.208333) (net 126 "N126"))
  (pad "2" smd roundrect (at 1 0 90) (size 1.2 1.4) (layers "F.Cu" "F.Paste" "F.Mask") (roundrect_rratio 0.208333) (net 1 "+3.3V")))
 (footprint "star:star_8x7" (layer "F.Cu") (at 130.302 137.922 90)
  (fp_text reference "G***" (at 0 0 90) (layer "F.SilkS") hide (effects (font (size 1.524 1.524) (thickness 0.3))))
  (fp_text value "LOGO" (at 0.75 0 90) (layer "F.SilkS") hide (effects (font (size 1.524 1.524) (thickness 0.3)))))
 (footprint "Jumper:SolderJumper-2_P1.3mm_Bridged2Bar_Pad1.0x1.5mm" (layer "F.Cu") (at 98.806 131.826 90)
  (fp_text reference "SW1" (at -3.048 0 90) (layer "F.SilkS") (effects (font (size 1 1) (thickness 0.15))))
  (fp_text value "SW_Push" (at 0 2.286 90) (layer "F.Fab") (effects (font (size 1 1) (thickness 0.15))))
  (fp_poly (pts (xy -0.25 0.2) (xy 0.25 0.2) (xy 0.25 0.6) (xy -0.25 0.6)) (layer "F.Cu") (width 0) (fill solid))
  (fp_poly (pts (xy -0.25 -0.6) (xy 0.25 -0.6) (xy 0.25 -0.2) (xy -0.25 -0.2)) (layer "F.Cu") (width 0) (fill solid))
  (pad "1" smd rect (at -0.65 0 90) (size 1 1.5) (layers "F.Cu" "F.Mask") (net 126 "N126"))
  (pad "2" smd rect (at 0.65 0 90) (size 1 1.5) (layers "F.Cu" "F.Mask") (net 2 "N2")))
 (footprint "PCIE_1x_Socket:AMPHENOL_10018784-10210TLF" (layer "F.Cu") (at 93.98 78.486 90)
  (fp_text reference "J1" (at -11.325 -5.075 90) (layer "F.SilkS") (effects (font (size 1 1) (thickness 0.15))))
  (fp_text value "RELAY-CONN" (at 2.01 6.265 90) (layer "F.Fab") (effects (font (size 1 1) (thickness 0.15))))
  (pad "" np_thru_hole circle locked (at 9.15 0 90) (size 2.35 2.35) (drill 2.35) (layers *.Cu *.Mask))
  (pad "" np_thru_hole circle locked (at 0 0 90) (size 2.35 2.35) (drill 2.35) (layers *.Cu *.Mask))
  (pad "A1" thru_hole rect locked (at -11.65 -1.25 90) (size 1.208 1.208) (drill 0.7) (layers *.Cu *.Mask) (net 1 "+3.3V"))
  (pad "A2" thru_hole circle locked (at -10.65 -3.25 90) (size 1.208 1.208) (drill 0.7) (layers *.Cu *.Mask) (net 14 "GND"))
  (pad "A3" thru_hole circle locked (at -9.65 -1.25 90) (size 1.208 1.208) (drill 0.7) (layers *.Cu *.Mask) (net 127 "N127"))
  (pad "A4" thru_hole circle locked (at -8.65 -3.25 90) (size 1.208 1.208) (drill 0.7) (layers *.Cu *.Mask) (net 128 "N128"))
  (pad "A5" thru_hole circle locked (at -7.65 -1.25 90) (size 1.208 1.208) (drill 0.7) (layers *.Cu *.Mask) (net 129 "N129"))
  (pad "A6" thru_hole circle locked (at -6.65 -3.25 90) (size 1.208 1.208) (drill 0.7) (layers *.Cu *.Mask) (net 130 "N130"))
  (pad "A7" thru_hole circle locked (at -5.65 -1.25 90) (size 1.208 1.208) (drill 0.7) (layers *.Cu *.Mask) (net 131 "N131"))
  (pad "A8" thru_hole circle locked (at -4.65 -3.25 90) (size 1.208 1.208) (drill 0.7) (layers *.Cu *.Mask) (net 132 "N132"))
  (pad "A9" thru_hole circle locked (at -3.65 -1.25 90) (size 1.208 1.208) (drill 0.7) (layers *.Cu *.Mask) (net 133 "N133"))
  (pad "A10" thru_hole circle locked (at -2.65 -3.25 90) (size 1.208 1.208) (drill 0.7) (layers *.Cu *.Mask) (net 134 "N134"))
  (pad "A11" thru_hole circle locked (at -1.65 -1.25 90) (size 1.208 1.208) (drill 0.7) (layers *.Cu *.Mask) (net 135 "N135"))
  (pad "A12" thru_hole circle locked (at 1.35 -3.25 90) (size 1.208 1.208) (drill 0.7) (layers *.Cu *.Mask) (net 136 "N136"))
  (pad "A13" thru_hole circle locked (at 2.35 -1.25 90) (size 1.208 1.208) (drill 0.7) (layers *.Cu *.Mask) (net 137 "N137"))
  (pad "A14" thru_hole circle locked (at 3.35 -3.25 90) (size 1.208 1.208) (drill 0.7) (layers *.Cu *.Mask) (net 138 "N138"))
  (pad "A15" thru_hole circle locked (at 4.35 -1.25 90) (size 1.208 1.208) (drill 0.7) (layers *.Cu *.Mask) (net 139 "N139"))
  (pad "A16" thru_hole circle locked (at 5.35 -3.25 90) (size 1.208 1.208) (drill 0.7) (layers *.Cu *.Mask) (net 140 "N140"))
  (pad "A17" thru_hole circle locked (at 6.35 -1.25 90) (size 1.208 1.208) (drill 0.7) (layers *.Cu *.Mask) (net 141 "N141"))
  (pad "A18" thru_hole circle locked (at 7.35 -3.25 90) (size 1.208 1.208) (drill 0.7) (layers *.Cu *.Mask) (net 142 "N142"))
  (pad "B1" thru_hole rect locked (at -11.65 1.25 90) (size 1.208 1.208) (drill 0.7) (layers *.Cu *.Mask) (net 20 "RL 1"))
  (pad "B2" thru_hole circle locked (at -10.65 3.25 90) (size 1.208 1.208) (drill 0.7) (layers *.Cu *.Mask) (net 21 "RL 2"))
  (pad "B3" thru_hole circle locked (at -9.65 1.25 90) (size 1.208 1.208) (drill 0.7) (layers *.Cu *.Mask) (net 24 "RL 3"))
  (pad "B4" thru_hole circle locked (at -8.65 3.25 90) (size 1.208 1.208) (drill 0.7) (layers *.Cu *.Mask) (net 25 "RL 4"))
  (pad "B5" thru_hole circle locked (at -7.65 1.25 90) (size 1.208 1.208) (drill 0.7) (layers *.Cu *.Mask) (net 26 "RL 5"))
  (pad "B6" thru_hole circle locked (at -6.65 3.25 90) (size 1.208 1.208) (drill 0.7) (layers *.Cu *.Mask) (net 27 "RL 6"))
  (pad "B7" thru_hole circle locked (at -5.65 1.25 90) (size 1.208 1.208) (drill 0.7) (layers *.Cu *.Mask) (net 28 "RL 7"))
  (pad "B8" thru_hole circle locked (at -4.65 3.25 90) (size 1.208 1.208) (drill 0.7) (layers *.Cu *.Mask) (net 29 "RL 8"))
  (pad "B9" thru_hole circle locked (at -3.65 1.25 90) (size 1.208 1.208) (drill 0.7) (layers *.Cu *.Mask) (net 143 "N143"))
  (pad "B10" thru_hole circle locked (at -2.65 3.25 90) (size 1.208 1.208) (drill 0.7) (layers *.Cu *.Mask) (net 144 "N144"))
  (pad "B11" thru_hole circle locked (at -1.65 1.25 90) (size 1.208 1.208) (drill 0.7) (layers *.Cu *.Mask) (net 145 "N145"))
  (pad "B12" thru_hole circle locked (at 1.35 3.25 90) (size 1.208 1.208) (drill 0.7) (layers *.Cu *.Mask) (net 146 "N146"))
  (pad "B13" thru_hole circle locked (at 2.35 1.25 90) (size 1.208 1.208) (drill 0.7) (layers *.Cu *.Mask) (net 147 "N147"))
  (pad "B14" thru_hole circle locked (at 3.35 3.25 90) (size 1.208 1.208) (drill 0.7) (layers *.Cu *.Mask) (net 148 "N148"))
  (pad "B15" thru_hole circle locked (at 4.35 1.25 90) (size 1.208 1.208) (drill 0.7) (layers *.Cu *.Mask) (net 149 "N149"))
  (pad "B16" thru_hole circle locked (at 5.35 3.25 90) (size 1.208 1.208) (drill 0.7) (layers *.Cu *.Mask) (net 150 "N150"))
  (pad "B17" thru_hole circle locked (at 6.35 1.25 90) (size 1.208 1.208) (drill 0.7) (layers *.Cu *.Mask) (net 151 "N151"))
  (pad "B18" thru_hole circle locked (at 7.35 3.25 90) (size 1.208 1.208) (drill 0.7) (layers *.Cu *.Mask) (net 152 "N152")))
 (gr_rect (start 85.852 46.736) (end 147.828 152.654) (layer "Edge.Cuts") (width 0.1) (fill none))
 (segment (start 93.472 129.592) (end 93.472 135.128) (width 0.25) (layer "F.Cu") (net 1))
 (segment (start 117.41 137.668) (end 118.929 136.149) (width 0.25) (layer "F.Cu") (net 1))
 (segment (start 96.318 126.746) (end 93.472 129.592) (width 0.25) (layer "F.Cu") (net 1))
 (segment (start 96.318 130.52) (end 96.012 130.826) (width 0.25) (layer "F.Cu") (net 1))
 (segment (start 96.012 137.668) (end 117.41 137.668) (width 0.25) (layer "F.Cu") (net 1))
 (segment (start 93.472 135.128) (end 96.012 137.668) (width 0.25) (layer "F.Cu") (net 1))
 (segment (start 96.318 126.746) (end 96.318 130.52) (width 0.25) (layer "F.Cu") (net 1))
 (segment (start 99.163 94.131) (end 92.73 100.564) (width 0.25) (layer "B.Cu") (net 1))
 (segment (start 92.73 97.048) (end 92.73 95.992) (width 0.25) (layer "B.Cu") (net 1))
 (segment (start 99.314 92.456) (end 92.73 99.04) (width 0.254) (layer "B.Cu") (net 1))
 (segment (start 96.318 126.746) (end 96.318 125.782) (width 0.25) (layer "B.Cu") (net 1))
 (segment (start 112.106 53.85) (end 114.419805 53.85) (width 0.25) (layer "B.Cu") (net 1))
 (segment (start 114.419805 53.85) (end 115.035 54.465195) (width 0.25) (layer "B.Cu") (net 1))
 (segment (start 96.318 126.746) (end 95.504 126.746) (width 0.25) (layer "B.Cu") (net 1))
 (segment (start 121.686 90.644) (end 121.686 91.166) (width 0.254) (layer "B.Cu") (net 1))
 (segment (start 92.73 95.992) (end 92.73 90.136) (width 0.25) (layer "B.Cu") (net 1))
 (segment (start 134.64 73.118) (end 134.64 92.992) (width 0.25) (layer "B.Cu") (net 1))
 (segment (start 115.035 54.465195) (end 115.035 74.703) (width 0.25) (layer "B.Cu") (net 1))
 (segment (start 92.73 98.532) (end 92.73 98.572) (width 0.254) (layer "B.Cu") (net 1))
 (segment (start 96.318 126.746) (end 92.73 123.158) (width 0.25) (layer "B.Cu") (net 1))
 (segment (start 121.686 91.166) (end 120.396 92.456) (width 0.254) (layer "B.Cu") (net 1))
 (segment (start 101.64 88.138) (end 100.985 88.793) (width 0.25) (layer "B.Cu") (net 1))
 (segment (start 92.73 100.564) (end 92.73 99.294) (width 0.25) (layer "B.Cu") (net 1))
 (segment (start 134.64 92.992) (end 133.501 94.131) (width 0.25) (layer "B.Cu") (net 1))
 (segment (start 92.73 123.158) (end 92.73 100.564) (width 0.25) (layer "B.Cu") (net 1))
 (segment (start 133.501 94.131) (end 99.163 94.131) (width 0.25) (layer "B.Cu") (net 1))
 (segment (start 100.985 88.753) (end 115.035 74.703) (width 0.25) (layer "B.Cu") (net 1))
 (segment (start 100.985 88.793) (end 100.985 88.753) (width 0.25) (layer "B.Cu") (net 1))
 (segment (start 92.73 99.04) (end 92.73 99.294) (width 0.254) (layer "B.Cu") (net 1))
 (segment (start 92.73 98.572) (end 92.73 97.048) (width 0.25) (layer "B.Cu") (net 1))
 (segment (start 120.396 92.456) (end 99.314 92.456) (width 0.254) (layer "B.Cu") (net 1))
 (segment (start 100.985 88.793) (end 92.73 97.048) (width 0.25) (layer "B.Cu") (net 1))
 (segment (start 92.73 99.294) (end 92.73 98.572) (width 0.25) (layer "B.Cu") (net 1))
 (via (at 144.78 149.352) (size 4) (drill 2) (layers "F.Cu" "B.Cu") (free) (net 14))
 (via (at 109.59 106.286) (size 0.8) (drill 0.4) (layers "F.Cu" "B.Cu") (free) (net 14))
 (via (at 109.59 103.746) (size 0.8) (drill 0.4) (layers "F.Cu" "B.Cu") (free) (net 14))
 (via (at 121.655 95.491) (size 0.8) (drill 0.4) (layers "F.Cu" "B.Cu") (free) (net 14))
 (via (at 88.646 49.784) (size 4) (drill 2) (layers "F.Cu" "B.Cu") (free) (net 14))
 (via (at 101.092 140.462) (size 0.8) (drill 0.4) (layers "F.Cu" "B.Cu") (free) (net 14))
 (via (at 88.646 149.352) (size 4) (drill 2) (layers "F.Cu" "B.Cu") (free) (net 14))
 (via (at 115.305 100.571) (size 0.8) (drill 0.4) (layers "F.Cu" "B.Cu") (free) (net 14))
 (via (at 121.655 103.746) (size 0.8) (drill 0.4) (layers "F.Cu" "B.Cu") (free) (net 14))
 (via (at 92.71 140.716) (size 0.8) (drill 0.4) (layers "F.Cu" "B.Cu") (free) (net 14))
 (via (at 115.305 103.746) (size 0.8) (drill 0.4) (layers "F.Cu" "B.Cu") (free) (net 14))
 (via (at 108.32 140.576) (size 0.8) (drill 0.4) (layers "F.Cu" "B.Cu") (free) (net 14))
 (via (at 115.305 106.286) (size 0.8) (drill 0.4) (layers "F.Cu" "B.Cu") (free) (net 14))
 (via (at 121.655 106.286) (size 0.8) (drill 0.4) (layers "F.Cu" "B.Cu") (free) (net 14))
 (via (at 122.29 140.576) (size 0.8) (drill 0.4) (layers "F.Cu" "B.Cu") (free) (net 14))
 (via (at 145.034 49.784) (size 4) (drill 2) (layers "F.Cu" "B.Cu") (free) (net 14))
 (via (at 109.59 91.046) (size 0.8) (drill 0.4) (layers "F.Cu" "B.Cu") (free) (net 14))
 (via (at 109.59 100.571) (size 0.8) (drill 0.4) (layers "F.Cu" "B.Cu") (free) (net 14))
 (via (at 121.655 100.571) (size 0.8) (drill 0.4) (layers "F.Cu" "B.Cu") (free) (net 14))
 (via (at 115.305 140.576) (size 0.8) (drill 0.4) (layers "F.Cu" "B.Cu") (free) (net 14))
 (via (at 115.305 91.046) (size 0.8) (drill 0.4) (layers "F.Cu" "B.Cu") (free) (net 14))
 (segment (start 96.362 132.476) (end 98.806 132.476) (width 0.25) (layer "F.Cu") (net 126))
 (segment (start 96.012 132.826) (end 96.362 132.476) (width 0.25) (layer "F.Cu") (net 126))
 (segment (start 138.063 125.641) (end 136.958 126.746) (width 0.25) (layer "F.Cu") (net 17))
 (segment (start 124.186 86.644) (end 124.257 86.715) (width 0.25) (layer "F.Cu") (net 11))
 (segment (start 98.858 131.124) (end 98.806 131.176) (width 0.25) (layer "F.Cu") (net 2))
 (segment (start 98.858 126.746) (end 98.858 131.124) (width 0.25) (layer "F.Cu") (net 2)))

